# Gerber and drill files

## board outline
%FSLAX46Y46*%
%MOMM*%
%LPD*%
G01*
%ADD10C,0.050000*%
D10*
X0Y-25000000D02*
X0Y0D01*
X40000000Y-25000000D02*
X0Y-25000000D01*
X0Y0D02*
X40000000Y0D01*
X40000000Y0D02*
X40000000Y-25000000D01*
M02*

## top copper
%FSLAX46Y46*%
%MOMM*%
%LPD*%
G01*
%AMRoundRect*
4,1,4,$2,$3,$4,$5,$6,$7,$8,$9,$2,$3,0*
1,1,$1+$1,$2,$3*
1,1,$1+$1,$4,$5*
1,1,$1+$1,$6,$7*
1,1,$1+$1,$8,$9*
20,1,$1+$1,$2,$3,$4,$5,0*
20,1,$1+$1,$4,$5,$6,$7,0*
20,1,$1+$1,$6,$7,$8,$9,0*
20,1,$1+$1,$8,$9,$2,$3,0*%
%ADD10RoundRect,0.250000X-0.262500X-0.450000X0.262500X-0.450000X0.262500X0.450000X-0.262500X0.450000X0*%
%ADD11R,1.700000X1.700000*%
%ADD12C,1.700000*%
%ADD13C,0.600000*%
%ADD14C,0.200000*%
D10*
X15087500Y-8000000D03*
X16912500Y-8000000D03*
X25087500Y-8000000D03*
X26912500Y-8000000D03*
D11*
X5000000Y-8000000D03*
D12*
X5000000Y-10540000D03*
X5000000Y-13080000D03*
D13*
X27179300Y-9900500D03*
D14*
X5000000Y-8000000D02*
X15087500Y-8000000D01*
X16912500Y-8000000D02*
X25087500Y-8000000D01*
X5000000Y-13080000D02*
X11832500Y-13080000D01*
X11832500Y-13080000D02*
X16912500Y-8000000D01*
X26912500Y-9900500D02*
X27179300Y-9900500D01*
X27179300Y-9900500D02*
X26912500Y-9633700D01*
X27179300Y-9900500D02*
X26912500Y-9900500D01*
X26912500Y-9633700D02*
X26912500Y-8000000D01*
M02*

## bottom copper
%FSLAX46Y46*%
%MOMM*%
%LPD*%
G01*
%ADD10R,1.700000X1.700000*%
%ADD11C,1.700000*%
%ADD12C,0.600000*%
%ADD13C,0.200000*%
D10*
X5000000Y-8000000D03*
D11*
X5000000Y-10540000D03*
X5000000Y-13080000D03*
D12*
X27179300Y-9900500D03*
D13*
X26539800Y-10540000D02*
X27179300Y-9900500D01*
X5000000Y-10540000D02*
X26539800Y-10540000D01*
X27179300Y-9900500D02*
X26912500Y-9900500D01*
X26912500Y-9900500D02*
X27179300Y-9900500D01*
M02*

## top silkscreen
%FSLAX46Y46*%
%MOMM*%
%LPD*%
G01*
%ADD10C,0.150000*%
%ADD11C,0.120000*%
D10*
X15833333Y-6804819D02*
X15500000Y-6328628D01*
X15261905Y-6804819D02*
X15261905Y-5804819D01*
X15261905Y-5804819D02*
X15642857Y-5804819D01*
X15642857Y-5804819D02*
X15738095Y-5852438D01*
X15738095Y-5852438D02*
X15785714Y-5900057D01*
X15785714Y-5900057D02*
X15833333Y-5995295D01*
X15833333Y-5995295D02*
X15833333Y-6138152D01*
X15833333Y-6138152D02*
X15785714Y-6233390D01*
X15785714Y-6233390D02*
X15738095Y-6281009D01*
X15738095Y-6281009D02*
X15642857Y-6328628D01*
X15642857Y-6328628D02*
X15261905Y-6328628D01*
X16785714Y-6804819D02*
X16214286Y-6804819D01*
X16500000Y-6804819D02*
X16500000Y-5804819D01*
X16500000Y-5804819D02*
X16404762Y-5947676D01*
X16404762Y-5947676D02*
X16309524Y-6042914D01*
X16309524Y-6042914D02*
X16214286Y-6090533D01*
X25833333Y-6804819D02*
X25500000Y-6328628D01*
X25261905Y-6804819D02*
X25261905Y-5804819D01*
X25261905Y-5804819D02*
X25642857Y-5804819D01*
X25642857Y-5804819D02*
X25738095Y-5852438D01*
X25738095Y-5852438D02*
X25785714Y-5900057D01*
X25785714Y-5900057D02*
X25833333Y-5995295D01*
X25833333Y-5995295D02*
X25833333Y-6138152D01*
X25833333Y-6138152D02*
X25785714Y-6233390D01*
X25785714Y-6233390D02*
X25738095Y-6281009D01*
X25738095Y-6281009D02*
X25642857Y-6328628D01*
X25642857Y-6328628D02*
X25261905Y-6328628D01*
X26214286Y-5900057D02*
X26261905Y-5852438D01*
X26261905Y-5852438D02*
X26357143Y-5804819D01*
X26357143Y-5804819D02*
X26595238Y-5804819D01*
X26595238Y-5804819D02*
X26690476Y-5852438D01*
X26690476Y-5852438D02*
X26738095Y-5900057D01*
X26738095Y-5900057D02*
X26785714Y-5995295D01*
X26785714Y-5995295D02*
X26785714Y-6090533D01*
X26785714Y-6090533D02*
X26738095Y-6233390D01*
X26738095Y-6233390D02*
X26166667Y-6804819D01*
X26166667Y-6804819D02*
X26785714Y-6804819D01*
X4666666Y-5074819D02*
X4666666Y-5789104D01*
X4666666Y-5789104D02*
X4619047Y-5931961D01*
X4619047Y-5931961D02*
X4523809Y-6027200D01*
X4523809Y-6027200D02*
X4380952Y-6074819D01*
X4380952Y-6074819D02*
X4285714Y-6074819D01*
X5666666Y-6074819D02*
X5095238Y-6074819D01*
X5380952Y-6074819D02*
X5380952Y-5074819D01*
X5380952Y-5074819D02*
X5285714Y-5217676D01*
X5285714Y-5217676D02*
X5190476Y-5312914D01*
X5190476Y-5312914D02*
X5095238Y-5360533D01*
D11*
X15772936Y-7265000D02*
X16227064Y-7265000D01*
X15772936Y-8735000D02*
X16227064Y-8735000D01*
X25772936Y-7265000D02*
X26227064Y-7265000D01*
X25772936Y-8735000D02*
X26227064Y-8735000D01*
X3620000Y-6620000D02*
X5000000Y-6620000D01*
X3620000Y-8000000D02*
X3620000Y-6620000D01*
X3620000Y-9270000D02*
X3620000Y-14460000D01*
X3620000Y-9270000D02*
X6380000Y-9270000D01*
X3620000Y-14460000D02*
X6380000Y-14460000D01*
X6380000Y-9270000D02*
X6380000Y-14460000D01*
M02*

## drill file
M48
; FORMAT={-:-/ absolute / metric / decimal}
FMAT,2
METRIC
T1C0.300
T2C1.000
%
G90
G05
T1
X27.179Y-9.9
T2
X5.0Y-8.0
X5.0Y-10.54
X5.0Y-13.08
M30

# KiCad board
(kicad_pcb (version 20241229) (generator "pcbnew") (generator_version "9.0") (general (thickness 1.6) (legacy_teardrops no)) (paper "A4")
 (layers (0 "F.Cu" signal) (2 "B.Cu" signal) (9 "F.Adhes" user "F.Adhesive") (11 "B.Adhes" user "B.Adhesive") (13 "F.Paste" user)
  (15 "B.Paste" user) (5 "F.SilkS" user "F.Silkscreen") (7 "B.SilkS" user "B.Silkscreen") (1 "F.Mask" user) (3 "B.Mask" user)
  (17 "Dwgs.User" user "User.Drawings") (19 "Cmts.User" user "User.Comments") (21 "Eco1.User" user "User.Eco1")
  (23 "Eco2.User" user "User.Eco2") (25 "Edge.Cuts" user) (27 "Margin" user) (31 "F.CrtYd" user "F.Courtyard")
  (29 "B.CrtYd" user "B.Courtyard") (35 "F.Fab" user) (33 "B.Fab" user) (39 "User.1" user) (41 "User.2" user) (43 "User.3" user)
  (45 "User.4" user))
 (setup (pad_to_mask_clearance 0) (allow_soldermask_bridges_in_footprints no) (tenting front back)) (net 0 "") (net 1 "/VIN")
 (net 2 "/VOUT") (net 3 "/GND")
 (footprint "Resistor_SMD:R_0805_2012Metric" (layer "F.Cu") (at 16 8)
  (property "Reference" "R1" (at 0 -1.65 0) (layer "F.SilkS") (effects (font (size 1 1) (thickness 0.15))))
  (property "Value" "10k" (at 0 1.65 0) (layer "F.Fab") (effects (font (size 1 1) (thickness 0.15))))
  (fp_line (start -0.227064 -0.735) (end 0.227064 -0.735) (stroke (width 0.12) (type solid)) (layer "F.SilkS"))
  (fp_line (start -0.227064 0.735) (end 0.227064 0.735) (stroke (width 0.12) (type solid)) (layer "F.SilkS"))
  (pad "1" smd roundrect (at -0.9125 0) (size 1.025 1.4) (layers "F.Cu" "F.Mask" "F.Paste") (roundrect_rratio 0.243902) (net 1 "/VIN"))
  (pad "2" smd roundrect (at 0.9125 0) (size 1.025 1.4) (layers "F.Cu" "F.Mask" "F.Paste") (roundrect_rratio 0.243902) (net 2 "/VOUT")))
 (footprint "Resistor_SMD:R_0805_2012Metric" (layer "F.Cu") (at 26 8)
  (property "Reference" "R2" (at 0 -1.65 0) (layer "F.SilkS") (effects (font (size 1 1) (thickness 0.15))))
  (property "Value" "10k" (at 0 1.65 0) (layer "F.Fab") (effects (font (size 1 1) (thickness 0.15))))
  (fp_line (start -0.227064 -0.735) (end 0.227064 -0.735) (stroke (width 0.12) (type solid)) (layer "F.SilkS"))
  (fp_line (start -0.227064 0.735) (end 0.227064 0.735) (stroke (width 0.12) (type solid)) (layer "F.SilkS"))
  (pad "1" smd roundrect (at -0.9125 0) (size 1.025 1.4) (layers "F.Cu" "F.Mask" "F.Paste") (roundrect_rratio 0.243902) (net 2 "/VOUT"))
  (pad "2" smd roundrect (at 0.9125 0) (size 1.025 1.4) (layers "F.Cu" "F.Mask" "F.Paste") (roundrect_rratio 0.243902) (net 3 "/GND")))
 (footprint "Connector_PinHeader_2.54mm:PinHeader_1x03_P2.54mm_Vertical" (layer "F.Cu") (at 5 8)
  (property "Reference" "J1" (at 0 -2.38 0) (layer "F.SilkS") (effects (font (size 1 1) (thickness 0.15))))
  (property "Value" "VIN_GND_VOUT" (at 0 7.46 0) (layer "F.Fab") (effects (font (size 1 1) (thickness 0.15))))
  (fp_line (start -1.38 -1.38) (end 0 -1.38) (stroke (width 0.12) (type solid)) (layer "F.SilkS"))
  (fp_line (start -1.38 0) (end -1.38 -1.38) (stroke (width 0.12) (type solid)) (layer "F.SilkS"))
  (fp_line (start -1.38 1.27) (end -1.38 6.46) (stroke (width 0.12) (type solid)) (layer "F.SilkS"))
  (fp_line (start -1.38 1.27) (end 1.38 1.27) (stroke (width 0.12) (type solid)) (layer "F.SilkS"))
  (fp_line (start -1.38 6.46) (end 1.38 6.46) (stroke (width 0.12) (type solid)) (layer "F.SilkS"))
  (fp_line (start 1.38 1.27) (end 1.38 6.46) (stroke (width 0.12) (type solid)) (layer "F.SilkS"))
  (pad "1" thru_hole rect (at 0 0) (size 1.7 1.7) (drill 1) (layers "*.Cu" "*.Mask") (remove_unused_layers no) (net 1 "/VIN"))
  (pad "2" thru_hole circle (at 0 2.54) (size 1.7 1.7) (drill 1) (layers "*.Cu" "*.Mask") (remove_unused_layers no) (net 3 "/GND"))
  (pad "3" thru_hole circle (at 0 5.08) (size 1.7 1.7) (drill 1) (layers "*.Cu" "*.Mask") (remove_unused_layers no) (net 2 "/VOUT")))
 (gr_line (start 0 25) (end 0 0) (stroke (width 0.05) (type default)) (layer "Edge.Cuts"))
 (gr_line (start 40 25) (end 0 25) (stroke (width 0.05) (type default)) (layer "Edge.Cuts"))
 (gr_line (start 0 0) (end 40 0) (stroke (width 0.05) (type default)) (layer "Edge.Cuts"))
 (gr_line (start 40 0) (end 40 25) (stroke (width 0.05) (type default)) (layer "Edge.Cuts"))
 (segment (start 5 8) (end 15.0875 8) (width 0.2) (layer "F.Cu") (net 1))
 (segment (start 16.9125 8) (end 25.0875 8) (width 0.2) (layer "F.Cu") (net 2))
 (segment (start 5 13.08) (end 11.8325 13.08) (width 0.2) (layer "F.Cu") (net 2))
 (segment (start 11.8325 13.08) (end 16.9125 8) (width 0.2) (layer "F.Cu") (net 2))
 (segment (start 26.9125 9.9005) (end 27.1793 9.9005) (width 0.2) (layer "F.Cu") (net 3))
 (segment (start 27.1793 9.9005) (end 26.9125 9.6337) (width 0.2) (layer "F.Cu") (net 3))
 (segment (start 27.1793 9.9005) (end 26.9125 9.9005) (width 0.2) (layer "F.Cu") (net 3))
 (segment (start 26.9125 9.6337) (end 26.9125 8) (width 0.2) (layer "F.Cu") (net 3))
 (via (at 27.1793 9.9005) (size 0.6) (drill 0.3) (layers "F.Cu" "B.Cu") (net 3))
 (segment (start 26.5398 10.54) (end 27.1793 9.9005) (width 0.2) (layer "B.Cu") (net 3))
 (segment (start 5 10.54) (end 26.5398 10.54) (width 0.2) (layer "B.Cu") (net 3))
 (segment (start 27.1793 9.9005) (end 26.9125 9.9005) (width 0.2) (layer "B.Cu") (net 3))
 (segment (start 26.9125 9.9005) (end 27.1793 9.9005) (width 0.2) (layer "B.Cu") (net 3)))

